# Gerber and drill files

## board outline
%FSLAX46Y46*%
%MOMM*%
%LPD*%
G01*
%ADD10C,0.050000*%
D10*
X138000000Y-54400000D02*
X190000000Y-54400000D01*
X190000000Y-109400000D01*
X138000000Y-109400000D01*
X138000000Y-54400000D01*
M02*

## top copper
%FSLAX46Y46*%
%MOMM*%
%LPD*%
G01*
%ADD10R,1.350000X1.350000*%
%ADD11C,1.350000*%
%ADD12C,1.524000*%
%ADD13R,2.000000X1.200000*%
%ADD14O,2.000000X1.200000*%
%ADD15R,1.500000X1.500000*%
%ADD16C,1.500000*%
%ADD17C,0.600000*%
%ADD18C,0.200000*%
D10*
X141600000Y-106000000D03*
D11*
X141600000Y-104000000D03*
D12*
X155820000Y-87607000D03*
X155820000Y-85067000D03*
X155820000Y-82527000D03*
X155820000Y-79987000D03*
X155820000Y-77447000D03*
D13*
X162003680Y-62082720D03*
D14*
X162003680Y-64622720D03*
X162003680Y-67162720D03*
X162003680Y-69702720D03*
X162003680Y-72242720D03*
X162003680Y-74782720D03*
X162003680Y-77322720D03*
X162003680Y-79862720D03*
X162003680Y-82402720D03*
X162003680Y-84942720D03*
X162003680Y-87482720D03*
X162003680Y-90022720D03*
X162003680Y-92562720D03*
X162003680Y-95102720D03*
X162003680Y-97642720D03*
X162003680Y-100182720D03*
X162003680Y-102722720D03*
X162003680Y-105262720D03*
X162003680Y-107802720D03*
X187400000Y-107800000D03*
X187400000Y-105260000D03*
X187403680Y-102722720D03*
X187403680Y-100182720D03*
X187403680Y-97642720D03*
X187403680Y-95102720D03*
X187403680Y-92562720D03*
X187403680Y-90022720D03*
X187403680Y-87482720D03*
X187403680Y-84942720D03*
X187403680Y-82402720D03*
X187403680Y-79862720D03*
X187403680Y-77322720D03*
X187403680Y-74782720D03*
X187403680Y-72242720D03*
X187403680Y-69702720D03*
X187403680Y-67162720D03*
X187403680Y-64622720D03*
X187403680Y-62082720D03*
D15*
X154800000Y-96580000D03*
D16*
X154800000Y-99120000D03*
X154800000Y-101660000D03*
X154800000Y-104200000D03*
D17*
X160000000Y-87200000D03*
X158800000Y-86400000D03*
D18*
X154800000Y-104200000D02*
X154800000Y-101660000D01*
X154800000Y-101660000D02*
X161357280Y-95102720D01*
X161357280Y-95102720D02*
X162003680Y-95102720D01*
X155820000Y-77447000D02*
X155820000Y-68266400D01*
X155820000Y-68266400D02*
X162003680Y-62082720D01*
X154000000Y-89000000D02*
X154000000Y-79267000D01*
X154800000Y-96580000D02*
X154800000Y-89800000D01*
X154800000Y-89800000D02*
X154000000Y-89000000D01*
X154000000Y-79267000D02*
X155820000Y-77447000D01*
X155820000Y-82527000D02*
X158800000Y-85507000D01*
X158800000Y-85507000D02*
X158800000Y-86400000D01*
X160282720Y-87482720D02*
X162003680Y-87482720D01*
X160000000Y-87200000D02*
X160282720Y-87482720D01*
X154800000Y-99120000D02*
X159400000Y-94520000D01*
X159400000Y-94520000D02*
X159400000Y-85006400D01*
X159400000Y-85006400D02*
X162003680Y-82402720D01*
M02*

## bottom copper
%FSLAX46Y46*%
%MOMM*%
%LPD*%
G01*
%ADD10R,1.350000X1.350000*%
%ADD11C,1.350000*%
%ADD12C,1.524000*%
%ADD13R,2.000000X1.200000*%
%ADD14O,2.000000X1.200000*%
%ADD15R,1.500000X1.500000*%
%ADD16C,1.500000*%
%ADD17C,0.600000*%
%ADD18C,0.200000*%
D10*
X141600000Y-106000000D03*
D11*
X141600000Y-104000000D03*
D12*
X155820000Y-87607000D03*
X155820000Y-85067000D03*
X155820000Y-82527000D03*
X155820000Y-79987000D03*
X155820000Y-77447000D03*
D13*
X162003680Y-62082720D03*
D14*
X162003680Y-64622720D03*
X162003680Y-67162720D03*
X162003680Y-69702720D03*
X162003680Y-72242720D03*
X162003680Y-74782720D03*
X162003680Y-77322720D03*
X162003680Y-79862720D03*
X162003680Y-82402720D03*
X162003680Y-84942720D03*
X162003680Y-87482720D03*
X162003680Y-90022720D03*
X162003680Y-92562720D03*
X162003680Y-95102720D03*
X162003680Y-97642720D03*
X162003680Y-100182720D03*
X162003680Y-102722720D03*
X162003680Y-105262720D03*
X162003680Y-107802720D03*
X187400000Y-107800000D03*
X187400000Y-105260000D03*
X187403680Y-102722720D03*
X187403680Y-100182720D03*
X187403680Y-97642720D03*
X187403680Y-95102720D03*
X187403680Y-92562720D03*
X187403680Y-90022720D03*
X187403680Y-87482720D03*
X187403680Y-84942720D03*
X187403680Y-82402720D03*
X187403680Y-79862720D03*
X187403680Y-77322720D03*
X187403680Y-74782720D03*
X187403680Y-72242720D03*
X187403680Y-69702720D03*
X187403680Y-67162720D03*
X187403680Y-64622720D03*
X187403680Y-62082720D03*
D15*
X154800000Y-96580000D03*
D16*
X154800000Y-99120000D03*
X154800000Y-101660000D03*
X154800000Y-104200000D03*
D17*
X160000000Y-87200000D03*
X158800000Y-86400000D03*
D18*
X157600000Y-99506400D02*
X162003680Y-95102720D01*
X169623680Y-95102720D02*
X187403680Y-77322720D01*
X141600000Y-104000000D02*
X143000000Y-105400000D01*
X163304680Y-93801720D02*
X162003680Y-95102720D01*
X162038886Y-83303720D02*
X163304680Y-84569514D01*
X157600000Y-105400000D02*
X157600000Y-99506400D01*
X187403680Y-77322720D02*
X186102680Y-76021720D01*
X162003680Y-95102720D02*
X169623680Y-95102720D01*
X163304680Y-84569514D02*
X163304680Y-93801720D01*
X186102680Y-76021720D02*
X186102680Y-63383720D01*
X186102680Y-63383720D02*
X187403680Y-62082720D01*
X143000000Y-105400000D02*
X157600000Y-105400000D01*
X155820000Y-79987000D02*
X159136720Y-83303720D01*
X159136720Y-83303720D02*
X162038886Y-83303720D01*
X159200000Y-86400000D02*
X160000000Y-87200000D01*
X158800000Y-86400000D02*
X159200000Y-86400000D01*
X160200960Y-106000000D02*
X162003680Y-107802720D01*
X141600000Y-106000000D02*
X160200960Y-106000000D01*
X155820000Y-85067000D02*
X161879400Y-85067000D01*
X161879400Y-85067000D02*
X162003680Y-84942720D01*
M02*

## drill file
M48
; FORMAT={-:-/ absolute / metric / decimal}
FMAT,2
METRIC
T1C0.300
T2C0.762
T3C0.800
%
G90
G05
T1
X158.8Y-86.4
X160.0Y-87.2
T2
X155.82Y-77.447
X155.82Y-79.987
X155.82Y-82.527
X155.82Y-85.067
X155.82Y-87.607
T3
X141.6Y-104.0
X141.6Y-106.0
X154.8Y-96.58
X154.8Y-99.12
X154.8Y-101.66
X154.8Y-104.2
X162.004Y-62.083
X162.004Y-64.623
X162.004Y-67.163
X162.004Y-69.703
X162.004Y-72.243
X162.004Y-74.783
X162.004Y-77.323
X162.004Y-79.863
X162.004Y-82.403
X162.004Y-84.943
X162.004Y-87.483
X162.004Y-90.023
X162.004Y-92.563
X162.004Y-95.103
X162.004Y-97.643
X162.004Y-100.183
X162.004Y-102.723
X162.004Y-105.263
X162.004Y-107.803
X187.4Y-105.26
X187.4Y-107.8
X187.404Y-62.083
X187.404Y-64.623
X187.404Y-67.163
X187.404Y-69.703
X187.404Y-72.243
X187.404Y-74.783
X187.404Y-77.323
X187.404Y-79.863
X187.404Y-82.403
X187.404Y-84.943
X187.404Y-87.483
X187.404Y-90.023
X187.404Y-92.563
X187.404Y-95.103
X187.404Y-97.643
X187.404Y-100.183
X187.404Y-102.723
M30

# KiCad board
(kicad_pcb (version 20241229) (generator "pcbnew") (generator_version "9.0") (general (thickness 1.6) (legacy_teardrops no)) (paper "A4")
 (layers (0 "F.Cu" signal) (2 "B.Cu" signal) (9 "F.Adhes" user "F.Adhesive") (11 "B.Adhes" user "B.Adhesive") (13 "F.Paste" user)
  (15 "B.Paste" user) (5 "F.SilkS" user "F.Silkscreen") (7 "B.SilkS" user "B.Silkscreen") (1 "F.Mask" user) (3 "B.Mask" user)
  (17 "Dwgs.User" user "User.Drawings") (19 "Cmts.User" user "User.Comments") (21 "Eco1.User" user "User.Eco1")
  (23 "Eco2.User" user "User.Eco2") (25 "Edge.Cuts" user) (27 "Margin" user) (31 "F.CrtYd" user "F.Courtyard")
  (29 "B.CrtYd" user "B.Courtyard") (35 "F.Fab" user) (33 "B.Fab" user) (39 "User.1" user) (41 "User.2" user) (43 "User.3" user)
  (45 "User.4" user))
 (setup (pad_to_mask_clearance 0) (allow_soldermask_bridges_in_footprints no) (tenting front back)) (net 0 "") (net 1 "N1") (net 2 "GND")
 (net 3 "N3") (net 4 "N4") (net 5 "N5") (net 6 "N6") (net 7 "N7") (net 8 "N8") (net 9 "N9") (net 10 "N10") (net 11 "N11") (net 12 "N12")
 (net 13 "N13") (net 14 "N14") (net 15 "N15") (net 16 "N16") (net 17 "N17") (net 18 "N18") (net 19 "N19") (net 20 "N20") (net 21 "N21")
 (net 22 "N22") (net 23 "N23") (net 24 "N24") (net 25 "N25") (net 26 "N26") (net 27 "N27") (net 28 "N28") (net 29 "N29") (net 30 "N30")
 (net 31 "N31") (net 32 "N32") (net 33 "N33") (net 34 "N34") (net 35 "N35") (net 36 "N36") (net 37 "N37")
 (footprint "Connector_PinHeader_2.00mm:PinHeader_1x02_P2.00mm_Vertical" (layer "F.Cu") (at 141.6 106 180)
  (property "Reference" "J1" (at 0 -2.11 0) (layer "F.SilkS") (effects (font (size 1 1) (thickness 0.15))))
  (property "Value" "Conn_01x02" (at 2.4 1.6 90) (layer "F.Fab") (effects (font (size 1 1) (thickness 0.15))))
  (pad "1" thru_hole rect (at 0 0 180) (size 1.35 1.35) (drill 0.8) (layers "*.Cu" "*.Mask") (remove_unused_layers no) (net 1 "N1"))
  (pad "2" thru_hole circle (at 0 2 180) (size 1.35 1.35) (drill 0.8) (layers "*.Cu" "*.Mask") (remove_unused_layers no) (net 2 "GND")))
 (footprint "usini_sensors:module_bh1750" (layer "F.Cu") (at 155.82 77.447 180)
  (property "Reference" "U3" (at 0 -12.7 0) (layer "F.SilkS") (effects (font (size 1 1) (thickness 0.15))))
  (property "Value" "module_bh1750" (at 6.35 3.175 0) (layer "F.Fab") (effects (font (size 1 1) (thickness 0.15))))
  (pad "1" thru_hole circle (at 0 -10.16 180) (size 1.524 1.524) (drill 0.762) (layers "*.Cu" "*.Mask") (remove_unused_layers no)
   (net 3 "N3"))
  (pad "2" thru_hole circle (at 0 -7.62 180) (size 1.524 1.524) (drill 0.762) (layers "*.Cu" "*.Mask") (remove_unused_layers no)
   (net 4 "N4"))
  (pad "3" thru_hole circle (at 0 -5.08 180) (size 1.524 1.524) (drill 0.762) (layers "*.Cu" "*.Mask") (remove_unused_layers no)
   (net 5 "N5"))
  (pad "4" thru_hole circle (at 0 -2.54 180) (size 1.524 1.524) (drill 0.762) (layers "*.Cu" "*.Mask") (remove_unused_layers no)
   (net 2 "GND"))
  (pad "5" thru_hole circle (at 0 0 180) (size 1.524 1.524) (drill 0.762) (layers "*.Cu" "*.Mask") (remove_unused_layers no) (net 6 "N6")))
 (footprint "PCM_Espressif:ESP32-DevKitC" (layer "F.Cu") (at 162.00368 62.08272)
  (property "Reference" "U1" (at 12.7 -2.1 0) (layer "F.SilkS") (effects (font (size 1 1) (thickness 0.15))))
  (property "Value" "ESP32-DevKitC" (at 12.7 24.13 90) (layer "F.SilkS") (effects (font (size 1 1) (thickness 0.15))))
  (pad "1" thru_hole rect (at 0 0 270) (size 1.2 2) (drill 0.8) (layers "*.Cu" "*.Mask") (remove_unused_layers no) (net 6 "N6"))
  (pad "2" thru_hole oval (at 0 2.54 270) (size 1.2 2) (drill 0.8) (layers "*.Cu" "*.Mask") (remove_unused_layers no) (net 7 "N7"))
  (pad "3" thru_hole oval (at 0 5.08 270) (size 1.2 2) (drill 0.8) (layers "*.Cu" "*.Mask") (remove_unused_layers no) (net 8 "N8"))
  (pad "4" thru_hole oval (at 0 7.62 270) (size 1.2 2) (drill 0.8) (layers "*.Cu" "*.Mask") (remove_unused_layers no) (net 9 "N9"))
  (pad "5" thru_hole oval (at 0 10.16 270) (size 1.2 2) (drill 0.8) (layers "*.Cu" "*.Mask") (remove_unused_layers no) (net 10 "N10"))
  (pad "6" thru_hole oval (at 0 12.7 270) (size 1.2 2) (drill 0.8) (layers "*.Cu" "*.Mask") (remove_unused_layers no) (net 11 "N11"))
  (pad "7" thru_hole oval (at 0 15.24 270) (size 1.2 2) (drill 0.8) (layers "*.Cu" "*.Mask") (remove_unused_layers no) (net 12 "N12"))
  (pad "8" thru_hole oval (at 0 17.78 270) (size 1.2 2) (drill 0.8) (layers "*.Cu" "*.Mask") (remove_unused_layers no) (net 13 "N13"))
  (pad "9" thru_hole oval (at 0 20.32 270) (size 1.2 2) (drill 0.8) (layers "*.Cu" "*.Mask") (remove_unused_layers no) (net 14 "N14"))
  (pad "10" thru_hole oval (at 0 22.86 270) (size 1.2 2) (drill 0.8) (layers "*.Cu" "*.Mask") (remove_unused_layers no) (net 4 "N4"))
  (pad "11" thru_hole oval (at 0 25.4 270) (size 1.2 2) (drill 0.8) (layers "*.Cu" "*.Mask") (remove_unused_layers no) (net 5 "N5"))
  (pad "12" thru_hole oval (at 0 27.94 270) (size 1.2 2) (drill 0.8) (layers "*.Cu" "*.Mask") (remove_unused_layers no) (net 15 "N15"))
  (pad "13" thru_hole oval (at 0 30.48 270) (size 1.2 2) (drill 0.8) (layers "*.Cu" "*.Mask") (remove_unused_layers no) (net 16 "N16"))
  (pad "14" thru_hole oval (at 0 33.02 270) (size 1.2 2) (drill 0.8) (layers "*.Cu" "*.Mask") (remove_unused_layers no) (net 2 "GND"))
  (pad "15" thru_hole oval (at 0 35.56 270) (size 1.2 2) (drill 0.8) (layers "*.Cu" "*.Mask") (remove_unused_layers no) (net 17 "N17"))
  (pad "16" thru_hole oval (at 0 38.1 270) (size 1.2 2) (drill 0.8) (layers "*.Cu" "*.Mask") (remove_unused_layers no) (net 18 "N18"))
  (pad "17" thru_hole oval (at 0 40.64 270) (size 1.2 2) (drill 0.8) (layers "*.Cu" "*.Mask") (remove_unused_layers no) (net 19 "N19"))
  (pad "18" thru_hole oval (at 0 43.18 270) (size 1.2 2) (drill 0.8) (layers "*.Cu" "*.Mask") (remove_unused_layers no) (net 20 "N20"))
  (pad "19" thru_hole oval (at 0 45.72 270) (size 1.2 2) (drill 0.8) (layers "*.Cu" "*.Mask") (remove_unused_layers no) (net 1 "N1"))
  (pad "20" thru_hole oval (at 25.39632 45.71728 270) (size 1.2 2) (drill 0.8) (layers "*.Cu" "*.Mask") (remove_unused_layers no)
   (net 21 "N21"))
  (pad "21" thru_hole oval (at 25.39632 43.17728 270) (size 1.2 2) (drill 0.8) (layers "*.Cu" "*.Mask") (remove_unused_layers no)
   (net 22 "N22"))
  (pad "22" thru_hole oval (at 25.4 40.64 270) (size 1.2 2) (drill 0.8) (layers "*.Cu" "*.Mask") (remove_unused_layers no) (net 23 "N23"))
  (pad "23" thru_hole oval (at 25.4 38.1 270) (size 1.2 2) (drill 0.8) (layers "*.Cu" "*.Mask") (remove_unused_layers no) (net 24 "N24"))
  (pad "24" thru_hole oval (at 25.4 35.56 270) (size 1.2 2) (drill 0.8) (layers "*.Cu" "*.Mask") (remove_unused_layers no) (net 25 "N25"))
  (pad "25" thru_hole oval (at 25.4 33.02 270) (size 1.2 2) (drill 0.8) (layers "*.Cu" "*.Mask") (remove_unused_layers no) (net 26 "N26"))
  (pad "26" thru_hole oval (at 25.4 30.48 270) (size 1.2 2) (drill 0.8) (layers "*.Cu" "*.Mask") (remove_unused_layers no) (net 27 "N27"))
  (pad "27" thru_hole oval (at 25.4 27.94 270) (size 1.2 2) (drill 0.8) (layers "*.Cu" "*.Mask") (remove_unused_layers no) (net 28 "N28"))
  (pad "28" thru_hole oval (at 25.4 25.4 270) (size 1.2 2) (drill 0.8) (layers "*.Cu" "*.Mask") (remove_unused_layers no) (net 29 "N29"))
  (pad "29" thru_hole oval (at 25.4 22.86 270) (size 1.2 2) (drill 0.8) (layers "*.Cu" "*.Mask") (remove_unused_layers no) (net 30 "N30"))
  (pad "30" thru_hole oval (at 25.4 20.32 270) (size 1.2 2) (drill 0.8) (layers "*.Cu" "*.Mask") (remove_unused_layers no) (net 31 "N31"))
  (pad "31" thru_hole oval (at 25.4 17.78 270) (size 1.2 2) (drill 0.8) (layers "*.Cu" "*.Mask") (remove_unused_layers no) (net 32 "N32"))
  (pad "32" thru_hole oval (at 25.4 15.24 270) (size 1.2 2) (drill 0.8) (layers "*.Cu" "*.Mask") (remove_unused_layers no) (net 2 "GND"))
  (pad "33" thru_hole oval (at 25.4 12.7 270) (size 1.2 2) (drill 0.8) (layers "*.Cu" "*.Mask") (remove_unused_layers no) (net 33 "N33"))
  (pad "34" thru_hole oval (at 25.4 10.16 270) (size 1.2 2) (drill 0.8) (layers "*.Cu" "*.Mask") (remove_unused_layers no) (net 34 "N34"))
  (pad "35" thru_hole oval (at 25.4 7.62 270) (size 1.2 2) (drill 0.8) (layers "*.Cu" "*.Mask") (remove_unused_layers no) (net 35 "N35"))
  (pad "36" thru_hole oval (at 25.4 5.08 270) (size 1.2 2) (drill 0.8) (layers "*.Cu" "*.Mask") (remove_unused_layers no) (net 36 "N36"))
  (pad "37" thru_hole oval (at 25.4 2.54 270) (size 1.2 2) (drill 0.8) (layers "*.Cu" "*.Mask") (remove_unused_layers no) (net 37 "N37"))
  (pad "38" thru_hole oval (at 25.4 0 270) (size 1.2 2) (drill 0.8) (layers "*.Cu" "*.Mask") (remove_unused_layers no) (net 2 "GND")))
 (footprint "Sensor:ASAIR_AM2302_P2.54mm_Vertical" (layer "F.Cu") (at 154.8 96.58 -90)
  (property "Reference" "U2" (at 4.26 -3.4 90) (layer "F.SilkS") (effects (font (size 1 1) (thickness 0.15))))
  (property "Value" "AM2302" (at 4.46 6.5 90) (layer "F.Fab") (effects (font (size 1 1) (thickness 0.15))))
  (pad "1" thru_hole rect (at 0 0) (size 1.5 1.5) (drill 0.8) (layers "*.Cu" "*.Mask") (remove_unused_layers no) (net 6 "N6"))
  (pad "2" thru_hole circle (at 2.54 0) (size 1.5 1.5) (drill 0.8) (layers "*.Cu" "*.Mask") (remove_unused_layers no) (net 14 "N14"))
  (pad "3" thru_hole circle (at 5.08 0) (size 1.5 1.5) (drill 0.8) (layers "*.Cu" "*.Mask") (remove_unused_layers no) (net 2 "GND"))
  (pad "4" thru_hole circle (at 7.62 0) (size 1.5 1.5) (drill 0.8) (layers "*.Cu" "*.Mask") (remove_unused_layers no) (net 2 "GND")))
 (gr_rect (start 138 54.4) (end 190 109.4) (stroke (width 0.05) (type default)) (fill no) (layer "Edge.Cuts"))
 (segment (start 154.8 104.2) (end 154.8 101.66) (width 0.2) (layer "F.Cu") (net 2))
 (segment (start 154.8 101.66) (end 161.35728 95.10272) (width 0.2) (layer "F.Cu") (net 2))
 (segment (start 161.35728 95.10272) (end 162.00368 95.10272) (width 0.2) (layer "F.Cu") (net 2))
 (segment (start 157.6 99.5064) (end 162.00368 95.10272) (width 0.2) (layer "B.Cu") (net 2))
 (segment (start 169.62368 95.10272) (end 187.40368 77.32272) (width 0.2) (layer "B.Cu") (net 2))
 (segment (start 141.6 104) (end 143 105.4) (width 0.2) (layer "B.Cu") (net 2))
 (segment (start 163.30468 93.80172) (end 162.00368 95.10272) (width 0.2) (layer "B.Cu") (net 2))
 (segment (start 162.038886 83.30372) (end 163.30468 84.569514) (width 0.2) (layer "B.Cu") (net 2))
 (segment (start 157.6 105.4) (end 157.6 99.5064) (width 0.2) (layer "B.Cu") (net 2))
 (segment (start 187.40368 77.32272) (end 186.10268 76.02172) (width 0.2) (layer "B.Cu") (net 2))
 (segment (start 162.00368 95.10272) (end 169.62368 95.10272) (width 0.2) (layer "B.Cu") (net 2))
 (segment (start 163.30468 84.569514) (end 163.30468 93.80172) (width 0.2) (layer "B.Cu") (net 2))
 (segment (start 186.10268 76.02172) (end 186.10268 63.38372) (width 0.2) (layer "B.Cu") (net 2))
 (segment (start 186.10268 63.38372) (end 187.40368 62.08272) (width 0.2) (layer "B.Cu") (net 2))
 (segment (start 143 105.4) (end 157.6 105.4) (width 0.2) (layer "B.Cu") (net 2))
 (segment (start 155.82 79.987) (end 159.13672 83.30372) (width 0.2) (layer "B.Cu") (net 2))
 (segment (start 159.13672 83.30372) (end 162.038886 83.30372) (width 0.2) (layer "B.Cu") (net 2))
 (segment (start 155.82 77.447) (end 155.82 68.2664) (width 0.2) (layer "F.Cu") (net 6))
 (segment (start 155.82 68.2664) (end 162.00368 62.08272) (width 0.2) (layer "F.Cu") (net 6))
 (segment (start 154 89) (end 154 79.267) (width 0.2) (layer "F.Cu") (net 6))
 (segment (start 154.8 96.58) (end 154.8 89.8) (width 0.2) (layer "F.Cu") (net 6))
 (segment (start 154.8 89.8) (end 154 89) (width 0.2) (layer "F.Cu") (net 6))
 (segment (start 154 79.267) (end 155.82 77.447) (width 0.2) (layer "F.Cu") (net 6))
 (segment (start 155.82 82.527) (end 158.8 85.507) (width 0.2) (layer "F.Cu") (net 5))
 (segment (start 158.8 85.507) (end 158.8 86.4) (width 0.2) (layer "F.Cu") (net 5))
 (segment (start 160.28272 87.48272) (end 162.00368 87.48272) (width 0.2) (layer "F.Cu") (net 5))
 (segment (start 160 87.2) (end 160.28272 87.48272) (width 0.2) (layer "F.Cu") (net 5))
 (via (at 160 87.2) (size 0.6) (drill 0.3) (layers "F.Cu" "B.Cu") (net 5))
 (via (at 158.8 86.4) (size 0.6) (drill 0.3) (layers "F.Cu" "B.Cu") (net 5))
 (segment (start 159.2 86.4) (end 160 87.2) (width 0.2) (layer "B.Cu") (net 5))
 (segment (start 158.8 86.4) (end 159.2 86.4) (width 0.2) (layer "B.Cu") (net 5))
 (segment (start 160.20096 106) (end 162.00368 107.80272) (width 0.2) (layer "B.Cu") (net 1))
 (segment (start 141.6 106) (end 160.20096 106) (width 0.2) (layer "B.Cu") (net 1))
 (segment (start 155.82 85.067) (end 161.8794 85.067) (width 0.2) (layer "B.Cu") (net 4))
 (segment (start 161.8794 85.067) (end 162.00368 84.94272) (width 0.2) (layer "B.Cu") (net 4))
 (segment (start 154.8 99.12) (end 159.4 94.52) (width 0.2) (layer "F.Cu") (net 14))
 (segment (start 159.4 94.52) (end 159.4 85.0064) (width 0.2) (layer "F.Cu") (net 14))
 (segment (start 159.4 85.0064) (end 162.00368 82.40272) (width 0.2) (layer "F.Cu") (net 14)))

